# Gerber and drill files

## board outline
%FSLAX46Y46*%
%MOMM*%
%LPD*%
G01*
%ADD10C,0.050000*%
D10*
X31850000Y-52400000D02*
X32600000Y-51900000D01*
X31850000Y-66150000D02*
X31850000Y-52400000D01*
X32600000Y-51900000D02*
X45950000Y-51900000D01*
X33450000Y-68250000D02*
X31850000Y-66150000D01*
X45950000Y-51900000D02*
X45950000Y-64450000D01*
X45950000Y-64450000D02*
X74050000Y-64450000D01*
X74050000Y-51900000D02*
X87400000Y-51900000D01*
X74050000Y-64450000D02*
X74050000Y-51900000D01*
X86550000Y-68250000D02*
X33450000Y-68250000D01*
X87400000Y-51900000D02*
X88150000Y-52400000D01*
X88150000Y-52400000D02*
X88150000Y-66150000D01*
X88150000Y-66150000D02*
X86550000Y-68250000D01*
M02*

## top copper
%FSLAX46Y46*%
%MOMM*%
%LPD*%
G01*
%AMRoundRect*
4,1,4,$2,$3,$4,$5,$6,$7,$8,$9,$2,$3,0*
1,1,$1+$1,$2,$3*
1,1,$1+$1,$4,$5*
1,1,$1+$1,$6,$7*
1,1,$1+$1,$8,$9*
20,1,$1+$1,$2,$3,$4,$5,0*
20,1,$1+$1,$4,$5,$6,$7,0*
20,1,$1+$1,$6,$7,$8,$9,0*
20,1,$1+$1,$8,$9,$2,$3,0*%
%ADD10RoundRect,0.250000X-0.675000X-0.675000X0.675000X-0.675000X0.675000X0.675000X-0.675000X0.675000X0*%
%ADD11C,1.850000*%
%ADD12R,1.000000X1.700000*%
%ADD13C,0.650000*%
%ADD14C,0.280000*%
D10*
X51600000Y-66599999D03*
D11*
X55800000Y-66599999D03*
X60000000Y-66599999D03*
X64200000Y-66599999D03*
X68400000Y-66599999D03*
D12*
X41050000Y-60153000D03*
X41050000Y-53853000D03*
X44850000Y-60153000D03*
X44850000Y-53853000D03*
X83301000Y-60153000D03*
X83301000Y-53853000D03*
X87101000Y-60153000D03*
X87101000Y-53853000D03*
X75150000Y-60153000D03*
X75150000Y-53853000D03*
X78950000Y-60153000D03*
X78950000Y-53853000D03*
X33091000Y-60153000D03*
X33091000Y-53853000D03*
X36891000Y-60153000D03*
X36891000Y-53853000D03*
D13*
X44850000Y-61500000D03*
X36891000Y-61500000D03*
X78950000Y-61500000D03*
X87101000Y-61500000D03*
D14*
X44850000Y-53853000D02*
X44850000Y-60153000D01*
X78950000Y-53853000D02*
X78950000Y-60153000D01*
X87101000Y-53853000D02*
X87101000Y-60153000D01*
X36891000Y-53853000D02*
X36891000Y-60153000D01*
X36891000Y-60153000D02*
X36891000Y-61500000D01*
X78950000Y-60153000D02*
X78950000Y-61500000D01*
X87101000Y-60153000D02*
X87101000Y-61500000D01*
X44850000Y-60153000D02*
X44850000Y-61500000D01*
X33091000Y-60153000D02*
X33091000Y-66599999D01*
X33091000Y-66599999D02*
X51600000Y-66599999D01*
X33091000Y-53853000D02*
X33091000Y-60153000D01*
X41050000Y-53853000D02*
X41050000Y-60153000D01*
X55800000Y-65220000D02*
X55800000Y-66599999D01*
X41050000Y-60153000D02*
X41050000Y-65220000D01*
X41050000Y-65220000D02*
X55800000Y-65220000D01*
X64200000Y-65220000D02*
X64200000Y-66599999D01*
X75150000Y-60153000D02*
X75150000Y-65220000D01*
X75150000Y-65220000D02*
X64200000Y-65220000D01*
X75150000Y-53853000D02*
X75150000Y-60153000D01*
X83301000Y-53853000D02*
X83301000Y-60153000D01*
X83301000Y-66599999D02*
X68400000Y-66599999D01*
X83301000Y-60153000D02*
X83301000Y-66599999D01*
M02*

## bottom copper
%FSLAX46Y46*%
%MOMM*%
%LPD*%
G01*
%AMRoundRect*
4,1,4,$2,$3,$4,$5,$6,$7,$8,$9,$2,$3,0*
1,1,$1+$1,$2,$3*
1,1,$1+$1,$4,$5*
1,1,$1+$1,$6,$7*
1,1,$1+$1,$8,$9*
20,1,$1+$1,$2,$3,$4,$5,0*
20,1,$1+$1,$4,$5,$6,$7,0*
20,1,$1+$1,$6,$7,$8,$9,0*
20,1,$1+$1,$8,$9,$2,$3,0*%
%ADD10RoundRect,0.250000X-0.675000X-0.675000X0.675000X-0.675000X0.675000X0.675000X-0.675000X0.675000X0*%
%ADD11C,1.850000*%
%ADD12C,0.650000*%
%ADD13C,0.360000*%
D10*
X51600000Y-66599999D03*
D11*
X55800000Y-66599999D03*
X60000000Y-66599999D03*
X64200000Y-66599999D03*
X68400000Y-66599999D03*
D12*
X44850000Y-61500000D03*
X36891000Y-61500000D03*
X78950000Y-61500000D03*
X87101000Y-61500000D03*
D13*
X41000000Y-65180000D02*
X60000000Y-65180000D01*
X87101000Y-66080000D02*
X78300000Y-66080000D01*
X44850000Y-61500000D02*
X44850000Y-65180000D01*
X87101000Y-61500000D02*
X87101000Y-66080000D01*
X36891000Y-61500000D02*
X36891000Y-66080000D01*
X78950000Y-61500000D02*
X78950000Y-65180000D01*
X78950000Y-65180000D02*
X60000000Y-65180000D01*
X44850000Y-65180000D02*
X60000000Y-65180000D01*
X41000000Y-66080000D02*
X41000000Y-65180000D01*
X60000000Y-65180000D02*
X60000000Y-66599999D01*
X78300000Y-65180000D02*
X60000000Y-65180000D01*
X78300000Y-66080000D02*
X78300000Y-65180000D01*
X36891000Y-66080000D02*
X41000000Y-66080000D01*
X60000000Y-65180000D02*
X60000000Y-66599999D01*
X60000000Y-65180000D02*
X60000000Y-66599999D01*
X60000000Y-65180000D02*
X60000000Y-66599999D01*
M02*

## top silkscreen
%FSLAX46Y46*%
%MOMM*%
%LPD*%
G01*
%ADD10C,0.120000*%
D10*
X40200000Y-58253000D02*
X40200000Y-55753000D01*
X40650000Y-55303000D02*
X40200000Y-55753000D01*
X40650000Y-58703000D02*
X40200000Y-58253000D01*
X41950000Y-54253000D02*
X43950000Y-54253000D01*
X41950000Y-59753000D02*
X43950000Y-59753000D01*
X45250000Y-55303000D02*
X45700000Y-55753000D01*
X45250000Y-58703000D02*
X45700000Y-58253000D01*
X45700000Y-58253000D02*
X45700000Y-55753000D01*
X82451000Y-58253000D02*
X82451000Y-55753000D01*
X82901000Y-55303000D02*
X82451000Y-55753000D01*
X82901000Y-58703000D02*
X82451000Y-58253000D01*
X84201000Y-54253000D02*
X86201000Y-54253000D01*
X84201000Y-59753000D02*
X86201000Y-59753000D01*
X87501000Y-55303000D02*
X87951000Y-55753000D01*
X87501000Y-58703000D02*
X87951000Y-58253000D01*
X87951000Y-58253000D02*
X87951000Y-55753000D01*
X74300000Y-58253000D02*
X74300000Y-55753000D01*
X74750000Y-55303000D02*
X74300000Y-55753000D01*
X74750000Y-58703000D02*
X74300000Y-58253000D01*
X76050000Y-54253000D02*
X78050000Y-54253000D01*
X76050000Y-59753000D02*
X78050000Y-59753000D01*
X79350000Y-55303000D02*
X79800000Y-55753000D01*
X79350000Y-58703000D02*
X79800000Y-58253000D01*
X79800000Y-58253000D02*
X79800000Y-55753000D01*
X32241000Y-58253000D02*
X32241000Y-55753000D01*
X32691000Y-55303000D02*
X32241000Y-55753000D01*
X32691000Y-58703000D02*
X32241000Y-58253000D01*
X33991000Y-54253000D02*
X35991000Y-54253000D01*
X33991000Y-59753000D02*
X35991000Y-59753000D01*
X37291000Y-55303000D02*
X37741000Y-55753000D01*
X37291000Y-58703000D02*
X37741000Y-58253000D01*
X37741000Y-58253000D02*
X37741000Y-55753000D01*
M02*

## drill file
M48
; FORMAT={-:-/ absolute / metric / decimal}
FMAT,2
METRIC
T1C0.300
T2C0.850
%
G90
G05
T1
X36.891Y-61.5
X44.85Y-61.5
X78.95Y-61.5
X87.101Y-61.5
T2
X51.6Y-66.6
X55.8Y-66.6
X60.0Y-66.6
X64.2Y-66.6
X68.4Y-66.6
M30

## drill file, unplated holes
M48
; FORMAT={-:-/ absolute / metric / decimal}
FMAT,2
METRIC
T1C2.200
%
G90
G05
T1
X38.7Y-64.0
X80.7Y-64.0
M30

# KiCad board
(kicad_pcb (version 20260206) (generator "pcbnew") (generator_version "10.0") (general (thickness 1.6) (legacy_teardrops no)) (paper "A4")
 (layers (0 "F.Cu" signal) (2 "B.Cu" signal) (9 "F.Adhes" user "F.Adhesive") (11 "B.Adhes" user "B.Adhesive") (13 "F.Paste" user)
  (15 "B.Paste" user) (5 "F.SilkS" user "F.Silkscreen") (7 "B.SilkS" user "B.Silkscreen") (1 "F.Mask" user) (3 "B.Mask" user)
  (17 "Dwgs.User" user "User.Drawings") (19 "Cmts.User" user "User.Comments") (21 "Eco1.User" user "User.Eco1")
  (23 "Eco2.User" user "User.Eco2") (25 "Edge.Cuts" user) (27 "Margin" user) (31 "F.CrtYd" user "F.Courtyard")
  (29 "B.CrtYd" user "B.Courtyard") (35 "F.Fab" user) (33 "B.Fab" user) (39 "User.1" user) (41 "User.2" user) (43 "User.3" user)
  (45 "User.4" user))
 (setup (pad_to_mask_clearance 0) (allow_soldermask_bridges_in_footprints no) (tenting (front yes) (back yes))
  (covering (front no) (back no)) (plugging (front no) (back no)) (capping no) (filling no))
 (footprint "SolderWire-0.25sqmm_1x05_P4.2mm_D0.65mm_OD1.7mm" (layer "F.Cu") (at 51.6 66.599999)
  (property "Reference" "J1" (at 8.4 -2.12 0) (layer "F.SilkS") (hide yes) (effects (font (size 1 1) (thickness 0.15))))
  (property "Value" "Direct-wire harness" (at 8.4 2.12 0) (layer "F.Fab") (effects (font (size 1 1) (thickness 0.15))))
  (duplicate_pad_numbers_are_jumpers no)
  (pad "1" thru_hole roundrect (at 0 0) (size 1.85 1.85) (drill 0.85) (layers "*.Cu" "*.Mask") (remove_unused_layers no)
   (roundrect_rratio 0.135135) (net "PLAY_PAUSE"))
  (pad "2" thru_hole circle (at 4.2 0) (size 1.85 1.85) (drill 0.85) (layers "*.Cu" "*.Mask") (remove_unused_layers no) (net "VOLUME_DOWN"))
  (pad "3" thru_hole circle (at 8.4 0) (size 1.85 1.85) (drill 0.85) (layers "*.Cu" "*.Mask") (remove_unused_layers no) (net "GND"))
  (pad "4" thru_hole circle (at 12.6 0) (size 1.85 1.85) (drill 0.85) (layers "*.Cu" "*.Mask") (remove_unused_layers no) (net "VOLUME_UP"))
  (pad "5" thru_hole circle (at 16.8 0) (size 1.85 1.85) (drill 0.85) (layers "*.Cu" "*.Mask") (remove_unused_layers no) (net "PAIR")))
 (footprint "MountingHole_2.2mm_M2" (layer "F.Cu") (at 38.7 64)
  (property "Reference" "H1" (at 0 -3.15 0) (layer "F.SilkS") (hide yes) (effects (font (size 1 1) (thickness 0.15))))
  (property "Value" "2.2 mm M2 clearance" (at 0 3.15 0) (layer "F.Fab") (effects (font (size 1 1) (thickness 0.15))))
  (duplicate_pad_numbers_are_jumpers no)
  (pad "" np_thru_hole circle (at 0 0) (size 2.2 2.2) (drill 2.2) (layers "*.Cu" "*.Mask")))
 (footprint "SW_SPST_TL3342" (layer "F.Cu") (at 42.95 57.003 90)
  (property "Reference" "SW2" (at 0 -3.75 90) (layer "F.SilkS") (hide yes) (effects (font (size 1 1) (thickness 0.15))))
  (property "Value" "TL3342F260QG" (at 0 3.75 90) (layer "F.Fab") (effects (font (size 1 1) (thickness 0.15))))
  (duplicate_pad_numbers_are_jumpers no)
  (fp_line (start -1.25 -2.75) (end 1.25 -2.75) (stroke (width 0.12) (type solid)) (layer "F.SilkS"))
  (fp_line (start 1.7 -2.3) (end 1.25 -2.75) (stroke (width 0.12) (type solid)) (layer "F.SilkS"))
  (fp_line (start -1.7 -2.3) (end -1.25 -2.75) (stroke (width 0.12) (type solid)) (layer "F.SilkS"))
  (fp_line (start 2.75 -1) (end 2.75 1) (stroke (width 0.12) (type solid)) (layer "F.SilkS"))
  (fp_line (start -2.75 -1) (end -2.75 1) (stroke (width 0.12) (type solid)) (layer "F.SilkS"))
  (fp_line (start 1.7 2.3) (end 1.25 2.75) (stroke (width 0.12) (type solid)) (layer "F.SilkS"))
  (fp_line (start -1.7 2.3) (end -1.25 2.75) (stroke (width 0.12) (type solid)) (layer "F.SilkS"))
  (fp_line (start -1.25 2.75) (end 1.25 2.75) (stroke (width 0.12) (type solid)) (layer "F.SilkS"))
  (pad "1" smd rect (at -3.15 -1.9 90) (size 1.7 1) (layers "F.Cu" "F.Mask" "F.Paste") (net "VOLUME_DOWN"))
  (pad "1" smd rect (at 3.15 -1.9 90) (size 1.7 1) (layers "F.Cu" "F.Mask" "F.Paste") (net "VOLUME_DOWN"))
  (pad "2" smd rect (at -3.15 1.9 90) (size 1.7 1) (layers "F.Cu" "F.Mask" "F.Paste") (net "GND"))
  (pad "2" smd rect (at 3.15 1.9 90) (size 1.7 1) (layers "F.Cu" "F.Mask" "F.Paste") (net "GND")))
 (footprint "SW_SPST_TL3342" (layer "F.Cu") (at 85.201 57.003 90)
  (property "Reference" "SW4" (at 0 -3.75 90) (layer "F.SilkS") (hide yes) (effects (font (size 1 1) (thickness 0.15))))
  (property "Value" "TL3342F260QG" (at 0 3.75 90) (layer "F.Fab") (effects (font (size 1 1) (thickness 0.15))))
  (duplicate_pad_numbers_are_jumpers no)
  (fp_line (start -1.25 -2.75) (end 1.25 -2.75) (stroke (width 0.12) (type solid)) (layer "F.SilkS"))
  (fp_line (start 1.7 -2.3) (end 1.25 -2.75) (stroke (width 0.12) (type solid)) (layer "F.SilkS"))
  (fp_line (start -1.7 -2.3) (end -1.25 -2.75) (stroke (width 0.12) (type solid)) (layer "F.SilkS"))
  (fp_line (start 2.75 -1) (end 2.75 1) (stroke (width 0.12) (type solid)) (layer "F.SilkS"))
  (fp_line (start -2.75 -1) (end -2.75 1) (stroke (width 0.12) (type solid)) (layer "F.SilkS"))
  (fp_line (start 1.7 2.3) (end 1.25 2.75) (stroke (width 0.12) (type solid)) (layer "F.SilkS"))
  (fp_line (start -1.7 2.3) (end -1.25 2.75) (stroke (width 0.12) (type solid)) (layer "F.SilkS"))
  (fp_line (start -1.25 2.75) (end 1.25 2.75) (stroke (width 0.12) (type solid)) (layer "F.SilkS"))
  (pad "1" smd rect (at -3.15 -1.9 90) (size 1.7 1) (layers "F.Cu" "F.Mask" "F.Paste") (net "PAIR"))
  (pad "1" smd rect (at 3.15 -1.9 90) (size 1.7 1) (layers "F.Cu" "F.Mask" "F.Paste") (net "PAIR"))
  (pad "2" smd rect (at -3.15 1.9 90) (size 1.7 1) (layers "F.Cu" "F.Mask" "F.Paste") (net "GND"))
  (pad "2" smd rect (at 3.15 1.9 90) (size 1.7 1) (layers "F.Cu" "F.Mask" "F.Paste") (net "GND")))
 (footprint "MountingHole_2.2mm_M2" (layer "F.Cu") (at 80.7 64)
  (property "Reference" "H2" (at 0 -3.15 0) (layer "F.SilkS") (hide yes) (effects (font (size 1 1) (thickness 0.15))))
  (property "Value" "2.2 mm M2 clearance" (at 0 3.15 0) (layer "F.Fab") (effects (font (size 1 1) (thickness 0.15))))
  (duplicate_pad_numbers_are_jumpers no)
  (pad "" np_thru_hole circle (at 0 0) (size 2.2 2.2) (drill 2.2) (layers "*.Cu" "*.Mask")))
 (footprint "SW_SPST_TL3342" (layer "F.Cu") (at 77.05 57.003 90)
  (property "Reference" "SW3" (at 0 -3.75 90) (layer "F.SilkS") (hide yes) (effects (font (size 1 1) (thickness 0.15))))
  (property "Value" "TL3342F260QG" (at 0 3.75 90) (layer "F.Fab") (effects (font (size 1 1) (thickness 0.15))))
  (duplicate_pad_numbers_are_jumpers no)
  (fp_line (start -1.25 -2.75) (end 1.25 -2.75) (stroke (width 0.12) (type solid)) (layer "F.SilkS"))
  (fp_line (start 1.7 -2.3) (end 1.25 -2.75) (stroke (width 0.12) (type solid)) (layer "F.SilkS"))
  (fp_line (start -1.7 -2.3) (end -1.25 -2.75) (stroke (width 0.12) (type solid)) (layer "F.SilkS"))
  (fp_line (start 2.75 -1) (end 2.75 1) (stroke (width 0.12) (type solid)) (layer "F.SilkS"))
  (fp_line (start -2.75 -1) (end -2.75 1) (stroke (width 0.12) (type solid)) (layer "F.SilkS"))
  (fp_line (start 1.7 2.3) (end 1.25 2.75) (stroke (width 0.12) (type solid)) (layer "F.SilkS"))
  (fp_line (start -1.7 2.3) (end -1.25 2.75) (stroke (width 0.12) (type solid)) (layer "F.SilkS"))
  (fp_line (start -1.25 2.75) (end 1.25 2.75) (stroke (width 0.12) (type solid)) (layer "F.SilkS"))
  (pad "1" smd rect (at -3.15 -1.9 90) (size 1.7 1) (layers "F.Cu" "F.Mask" "F.Paste") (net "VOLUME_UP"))
  (pad "1" smd rect (at 3.15 -1.9 90) (size 1.7 1) (layers "F.Cu" "F.Mask" "F.Paste") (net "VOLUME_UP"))
  (pad "2" smd rect (at -3.15 1.9 90) (size 1.7 1) (layers "F.Cu" "F.Mask" "F.Paste") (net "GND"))
  (pad "2" smd rect (at 3.15 1.9 90) (size 1.7 1) (layers "F.Cu" "F.Mask" "F.Paste") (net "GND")))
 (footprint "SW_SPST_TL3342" (layer "F.Cu") (at 34.991 57.003 90)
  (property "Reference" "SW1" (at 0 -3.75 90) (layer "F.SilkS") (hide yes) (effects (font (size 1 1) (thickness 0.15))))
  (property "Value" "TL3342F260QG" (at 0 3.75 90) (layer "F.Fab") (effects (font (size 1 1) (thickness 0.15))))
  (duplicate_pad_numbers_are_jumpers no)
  (fp_line (start -1.25 -2.75) (end 1.25 -2.75) (stroke (width 0.12) (type solid)) (layer "F.SilkS"))
  (fp_line (start 1.7 -2.3) (end 1.25 -2.75) (stroke (width 0.12) (type solid)) (layer "F.SilkS"))
  (fp_line (start -1.7 -2.3) (end -1.25 -2.75) (stroke (width 0.12) (type solid)) (layer "F.SilkS"))
  (fp_line (start 2.75 -1) (end 2.75 1) (stroke (width 0.12) (type solid)) (layer "F.SilkS"))
  (fp_line (start -2.75 -1) (end -2.75 1) (stroke (width 0.12) (type solid)) (layer "F.SilkS"))
  (fp_line (start 1.7 2.3) (end 1.25 2.75) (stroke (width 0.12) (type solid)) (layer "F.SilkS"))
  (fp_line (start -1.7 2.3) (end -1.25 2.75) (stroke (width 0.12) (type solid)) (layer "F.SilkS"))
  (fp_line (start -1.25 2.75) (end 1.25 2.75) (stroke (width 0.12) (type solid)) (layer "F.SilkS"))
  (pad "1" smd rect (at -3.15 -1.9 90) (size 1.7 1) (layers "F.Cu" "F.Mask" "F.Paste") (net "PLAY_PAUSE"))
  (pad "1" smd rect (at 3.15 -1.9 90) (size 1.7 1) (layers "F.Cu" "F.Mask" "F.Paste") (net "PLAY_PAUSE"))
  (pad "2" smd rect (at -3.15 1.9 90) (size 1.7 1) (layers "F.Cu" "F.Mask" "F.Paste") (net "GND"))
  (pad "2" smd rect (at 3.15 1.9 90) (size 1.7 1) (layers "F.Cu" "F.Mask" "F.Paste") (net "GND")))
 (gr_line (start 31.85 52.4) (end 32.6 51.9) (stroke (width 0.05) (type default)) (layer "Edge.Cuts"))
 (gr_line (start 31.85 66.15) (end 31.85 52.4) (stroke (width 0.05) (type default)) (layer "Edge.Cuts"))
 (gr_line (start 32.6 51.9) (end 45.95 51.9) (stroke (width 0.05) (type default)) (layer "Edge.Cuts"))
 (gr_line (start 33.45 68.25) (end 31.85 66.15) (stroke (width 0.05) (type default)) (layer "Edge.Cuts"))
 (gr_line (start 45.95 51.9) (end 45.95 64.45) (stroke (width 0.05) (type default)) (layer "Edge.Cuts"))
 (gr_line (start 45.95 64.45) (end 74.05 64.45) (stroke (width 0.05) (type default)) (layer "Edge.Cuts"))
 (gr_line (start 74.05 51.9) (end 87.4 51.9) (stroke (width 0.05) (type default)) (layer "Edge.Cuts"))
 (gr_line (start 74.05 64.45) (end 74.05 51.9) (stroke (width 0.05) (type default)) (layer "Edge.Cuts"))
 (gr_line (start 86.55 68.25) (end 33.45 68.25) (stroke (width 0.05) (type default)) (layer "Edge.Cuts"))
 (gr_line (start 87.4 51.9) (end 88.15 52.4) (stroke (width 0.05) (type default)) (layer "Edge.Cuts"))
 (gr_line (start 88.15 52.4) (end 88.15 66.15) (stroke (width 0.05) (type default)) (layer "Edge.Cuts"))
 (gr_line (start 88.15 66.15) (end 86.55 68.25) (stroke (width 0.05) (type default)) (layer "Edge.Cuts"))
 (segment (start 44.85 53.853) (end 44.85 60.153) (width 0.28) (layer "F.Cu") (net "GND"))
 (segment (start 78.95 53.853) (end 78.95 60.153) (width 0.28) (layer "F.Cu") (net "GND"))
 (segment (start 87.101 53.853) (end 87.101 60.153) (width 0.28) (layer "F.Cu") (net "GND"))
 (segment (start 36.891 53.853) (end 36.891 60.153) (width 0.28) (layer "F.Cu") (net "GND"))
 (segment (start 36.891 60.153) (end 36.891 61.5) (width 0.28) (layer "F.Cu") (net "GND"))
 (segment (start 78.95 60.153) (end 78.95 61.5) (width 0.28) (layer "F.Cu") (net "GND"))
 (segment (start 87.101 60.153) (end 87.101 61.5) (width 0.28) (layer "F.Cu") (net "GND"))
 (segment (start 44.85 60.153) (end 44.85 61.5) (width 0.28) (layer "F.Cu") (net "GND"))
 (via (at 44.85 61.5) (size 0.65) (drill 0.3) (layers "F.Cu" "B.Cu") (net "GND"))
 (via (at 36.891 61.5) (size 0.65) (drill 0.3) (layers "F.Cu" "B.Cu") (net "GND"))
 (via (at 78.95 61.5) (size 0.65) (drill 0.3) (layers "F.Cu" "B.Cu") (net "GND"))
 (via (at 87.101 61.5) (size 0.65) (drill 0.3) (layers "F.Cu" "B.Cu") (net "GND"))
 (segment (start 41 65.18) (end 60 65.18) (width 0.36) (layer "B.Cu") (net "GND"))
 (segment (start 87.101 66.08) (end 78.3 66.08) (width 0.36) (layer "B.Cu") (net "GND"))
 (segment (start 44.85 61.5) (end 44.85 65.18) (width 0.36) (layer "B.Cu") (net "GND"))
 (segment (start 87.101 61.5) (end 87.101 66.08) (width 0.36) (layer "B.Cu") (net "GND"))
 (segment (start 36.891 61.5) (end 36.891 66.08) (width 0.36) (layer "B.Cu") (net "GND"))
 (segment (start 78.95 61.5) (end 78.95 65.18) (width 0.36) (layer "B.Cu") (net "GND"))
 (segment (start 78.95 65.18) (end 60 65.18) (width 0.36) (layer "B.Cu") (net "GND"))
 (segment (start 44.85 65.18) (end 60 65.18) (width 0.36) (layer "B.Cu") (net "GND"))
 (segment (start 41 66.08) (end 41 65.18) (width 0.36) (layer "B.Cu") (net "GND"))
 (segment (start 60 65.18) (end 60 66.599999) (width 0.36) (layer "B.Cu") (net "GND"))
 (segment (start 78.3 65.18) (end 60 65.18) (width 0.36) (layer "B.Cu") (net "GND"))
 (segment (start 78.3 66.08) (end 78.3 65.18) (width 0.36) (layer "B.Cu") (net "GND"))
 (segment (start 36.891 66.08) (end 41 66.08) (width 0.36) (layer "B.Cu") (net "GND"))
 (segment (start 60 65.18) (end 60 66.599999) (width 0.36) (layer "B.Cu") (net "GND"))
 (segment (start 60 65.18) (end 60 66.599999) (width 0.36) (layer "B.Cu") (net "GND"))
 (segment (start 60 65.18) (end 60 66.599999) (width 0.36) (layer "B.Cu") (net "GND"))
 (segment (start 33.091 60.153) (end 33.091 66.599999) (width 0.28) (layer "F.Cu") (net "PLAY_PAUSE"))
 (segment (start 33.091 66.599999) (end 51.6 66.599999) (width 0.28) (layer "F.Cu") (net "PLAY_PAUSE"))
 (segment (start 33.091 53.853) (end 33.091 60.153) (width 0.28) (layer "F.Cu") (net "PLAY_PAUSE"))
 (segment (start 41.05 53.853) (end 41.05 60.153) (width 0.28) (layer "F.Cu") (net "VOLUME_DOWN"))
 (segment (start 55.8 65.22) (end 55.8 66.599999) (width 0.28) (layer "F.Cu") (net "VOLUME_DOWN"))
 (segment (start 41.05 60.153) (end 41.05 65.22) (width 0.28) (layer "F.Cu") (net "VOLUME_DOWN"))
 (segment (start 41.05 65.22) (end 55.8 65.22) (width 0.28) (layer "F.Cu") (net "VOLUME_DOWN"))
 (segment (start 64.2 65.22) (end 64.2 66.599999) (width 0.28) (layer "F.Cu") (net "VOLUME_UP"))
 (segment (start 75.15 60.153) (end 75.15 65.22) (width 0.28) (layer "F.Cu") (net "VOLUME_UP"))
 (segment (start 75.15 65.22) (end 64.2 65.22) (width 0.28) (layer "F.Cu") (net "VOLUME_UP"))
 (segment (start 75.15 53.853) (end 75.15 60.153) (width 0.28) (layer "F.Cu") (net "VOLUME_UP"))
 (segment (start 83.301 53.853) (end 83.301 60.153) (width 0.28) (layer "F.Cu") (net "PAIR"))
 (segment (start 83.301 66.599999) (end 68.4 66.599999) (width 0.28) (layer "F.Cu") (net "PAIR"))
 (segment (start 83.301 60.153) (end 83.301 66.599999) (width 0.28) (layer "F.Cu") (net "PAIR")))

